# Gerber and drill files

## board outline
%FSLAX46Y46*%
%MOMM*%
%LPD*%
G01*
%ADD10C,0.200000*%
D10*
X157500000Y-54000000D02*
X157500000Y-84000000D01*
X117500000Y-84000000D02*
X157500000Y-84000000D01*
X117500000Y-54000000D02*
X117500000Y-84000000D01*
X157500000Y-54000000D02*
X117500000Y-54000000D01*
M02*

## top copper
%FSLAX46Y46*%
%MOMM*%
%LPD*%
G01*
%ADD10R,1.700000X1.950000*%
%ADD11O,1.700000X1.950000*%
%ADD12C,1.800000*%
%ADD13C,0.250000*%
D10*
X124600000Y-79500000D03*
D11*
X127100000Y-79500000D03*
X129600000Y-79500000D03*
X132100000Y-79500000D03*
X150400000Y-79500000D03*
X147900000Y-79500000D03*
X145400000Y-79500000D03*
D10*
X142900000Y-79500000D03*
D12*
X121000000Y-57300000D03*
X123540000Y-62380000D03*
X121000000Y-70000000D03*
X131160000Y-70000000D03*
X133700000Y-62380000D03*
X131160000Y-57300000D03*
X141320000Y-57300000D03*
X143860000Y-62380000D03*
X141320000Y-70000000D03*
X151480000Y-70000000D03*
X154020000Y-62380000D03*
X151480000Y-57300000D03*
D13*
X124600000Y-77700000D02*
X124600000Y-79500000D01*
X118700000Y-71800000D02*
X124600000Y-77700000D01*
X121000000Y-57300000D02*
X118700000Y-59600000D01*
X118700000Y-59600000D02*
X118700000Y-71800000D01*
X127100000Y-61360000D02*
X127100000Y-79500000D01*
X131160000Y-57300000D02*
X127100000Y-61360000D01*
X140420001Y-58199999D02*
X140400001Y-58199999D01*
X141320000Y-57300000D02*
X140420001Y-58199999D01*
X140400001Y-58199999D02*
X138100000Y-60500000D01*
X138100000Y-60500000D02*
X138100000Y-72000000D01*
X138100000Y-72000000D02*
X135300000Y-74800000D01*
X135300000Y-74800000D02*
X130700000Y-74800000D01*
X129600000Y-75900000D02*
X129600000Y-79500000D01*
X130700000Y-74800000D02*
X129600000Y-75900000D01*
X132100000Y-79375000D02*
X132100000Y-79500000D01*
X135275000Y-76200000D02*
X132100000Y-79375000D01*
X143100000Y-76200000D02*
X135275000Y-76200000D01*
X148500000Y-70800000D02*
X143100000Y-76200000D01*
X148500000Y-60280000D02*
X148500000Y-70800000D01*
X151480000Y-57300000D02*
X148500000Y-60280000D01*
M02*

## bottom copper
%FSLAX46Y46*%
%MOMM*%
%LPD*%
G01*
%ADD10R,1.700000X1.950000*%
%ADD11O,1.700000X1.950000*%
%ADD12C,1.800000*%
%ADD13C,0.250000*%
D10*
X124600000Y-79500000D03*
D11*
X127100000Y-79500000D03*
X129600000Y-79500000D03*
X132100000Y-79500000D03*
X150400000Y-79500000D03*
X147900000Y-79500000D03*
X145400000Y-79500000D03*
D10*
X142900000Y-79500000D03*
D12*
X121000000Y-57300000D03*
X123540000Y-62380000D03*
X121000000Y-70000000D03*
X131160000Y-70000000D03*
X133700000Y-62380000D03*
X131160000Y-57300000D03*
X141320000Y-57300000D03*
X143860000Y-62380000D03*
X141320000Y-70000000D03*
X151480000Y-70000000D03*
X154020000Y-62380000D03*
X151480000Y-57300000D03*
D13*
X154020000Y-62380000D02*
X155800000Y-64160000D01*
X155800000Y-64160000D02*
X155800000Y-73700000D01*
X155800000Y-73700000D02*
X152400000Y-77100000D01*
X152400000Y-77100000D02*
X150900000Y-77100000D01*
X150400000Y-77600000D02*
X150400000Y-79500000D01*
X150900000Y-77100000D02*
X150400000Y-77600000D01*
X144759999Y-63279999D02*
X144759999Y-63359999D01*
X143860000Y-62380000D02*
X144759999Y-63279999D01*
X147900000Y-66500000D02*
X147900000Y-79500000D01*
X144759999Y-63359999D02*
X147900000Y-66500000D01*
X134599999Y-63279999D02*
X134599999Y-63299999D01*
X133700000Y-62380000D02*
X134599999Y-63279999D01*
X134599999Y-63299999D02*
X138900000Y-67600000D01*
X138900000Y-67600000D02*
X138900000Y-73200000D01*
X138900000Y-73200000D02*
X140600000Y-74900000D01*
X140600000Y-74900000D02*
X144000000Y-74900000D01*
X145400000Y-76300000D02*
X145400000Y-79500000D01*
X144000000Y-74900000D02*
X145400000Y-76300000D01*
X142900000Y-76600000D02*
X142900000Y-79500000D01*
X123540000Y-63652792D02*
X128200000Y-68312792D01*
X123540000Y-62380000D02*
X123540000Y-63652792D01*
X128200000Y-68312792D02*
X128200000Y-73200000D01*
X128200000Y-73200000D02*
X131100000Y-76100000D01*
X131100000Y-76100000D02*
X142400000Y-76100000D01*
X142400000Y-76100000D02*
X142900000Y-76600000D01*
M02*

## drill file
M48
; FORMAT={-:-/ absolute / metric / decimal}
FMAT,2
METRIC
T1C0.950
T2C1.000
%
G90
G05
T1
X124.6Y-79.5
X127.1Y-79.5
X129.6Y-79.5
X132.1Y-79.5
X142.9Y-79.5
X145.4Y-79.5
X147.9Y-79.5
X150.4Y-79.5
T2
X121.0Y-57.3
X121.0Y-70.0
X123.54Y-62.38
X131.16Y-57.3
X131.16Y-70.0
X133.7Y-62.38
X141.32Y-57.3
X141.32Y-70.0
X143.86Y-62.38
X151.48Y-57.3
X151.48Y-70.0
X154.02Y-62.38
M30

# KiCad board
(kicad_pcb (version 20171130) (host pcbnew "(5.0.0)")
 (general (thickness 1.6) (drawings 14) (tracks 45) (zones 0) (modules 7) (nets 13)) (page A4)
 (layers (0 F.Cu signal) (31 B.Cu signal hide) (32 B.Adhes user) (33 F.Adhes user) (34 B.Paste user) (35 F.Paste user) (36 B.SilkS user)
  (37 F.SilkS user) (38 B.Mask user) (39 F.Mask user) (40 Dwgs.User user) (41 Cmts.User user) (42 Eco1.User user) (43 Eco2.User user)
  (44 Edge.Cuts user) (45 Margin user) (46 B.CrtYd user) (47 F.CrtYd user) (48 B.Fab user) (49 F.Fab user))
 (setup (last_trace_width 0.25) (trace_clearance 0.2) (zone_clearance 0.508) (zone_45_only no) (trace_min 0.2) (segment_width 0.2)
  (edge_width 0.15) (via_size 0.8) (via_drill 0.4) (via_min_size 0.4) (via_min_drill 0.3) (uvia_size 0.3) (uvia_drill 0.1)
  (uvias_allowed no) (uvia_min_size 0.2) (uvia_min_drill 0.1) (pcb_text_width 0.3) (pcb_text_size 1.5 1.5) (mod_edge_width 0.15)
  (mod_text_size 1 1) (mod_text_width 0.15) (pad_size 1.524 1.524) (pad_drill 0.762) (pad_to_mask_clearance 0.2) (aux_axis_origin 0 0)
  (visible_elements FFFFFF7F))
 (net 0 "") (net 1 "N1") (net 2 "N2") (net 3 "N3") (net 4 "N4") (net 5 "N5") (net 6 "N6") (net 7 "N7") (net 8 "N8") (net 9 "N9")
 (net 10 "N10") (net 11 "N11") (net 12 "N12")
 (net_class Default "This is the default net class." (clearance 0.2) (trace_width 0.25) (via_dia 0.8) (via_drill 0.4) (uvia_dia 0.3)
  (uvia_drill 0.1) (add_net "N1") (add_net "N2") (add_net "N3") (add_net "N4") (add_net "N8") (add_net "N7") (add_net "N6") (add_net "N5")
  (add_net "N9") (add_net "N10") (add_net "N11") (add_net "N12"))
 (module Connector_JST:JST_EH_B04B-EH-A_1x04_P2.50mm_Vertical (layer F.Cu) (at 124.6 79.5)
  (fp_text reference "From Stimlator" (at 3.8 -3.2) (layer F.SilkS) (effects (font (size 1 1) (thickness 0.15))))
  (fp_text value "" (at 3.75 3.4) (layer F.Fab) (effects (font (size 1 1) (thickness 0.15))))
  (pad 1 thru_hole rect (at 0 0) (size 1.7 1.95) (drill 0.95) (layers *.Cu *.Mask) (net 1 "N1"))
  (pad 2 thru_hole oval (at 2.5 0) (size 1.7 1.95) (drill 0.95) (layers *.Cu *.Mask) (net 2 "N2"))
  (pad 3 thru_hole oval (at 5 0) (size 1.7 1.95) (drill 0.95) (layers *.Cu *.Mask) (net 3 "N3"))
  (pad 4 thru_hole oval (at 7.5 0) (size 1.7 1.95) (drill 0.95) (layers *.Cu *.Mask) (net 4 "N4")))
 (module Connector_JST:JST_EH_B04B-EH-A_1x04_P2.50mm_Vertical (layer F.Cu) (at 142.9 79.5)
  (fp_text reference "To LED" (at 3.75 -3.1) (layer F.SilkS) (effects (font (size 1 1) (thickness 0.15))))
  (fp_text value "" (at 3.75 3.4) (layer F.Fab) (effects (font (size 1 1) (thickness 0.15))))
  (pad 4 thru_hole oval (at 7.5 0) (size 1.7 1.95) (drill 0.95) (layers *.Cu *.Mask) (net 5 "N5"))
  (pad 3 thru_hole oval (at 5 0) (size 1.7 1.95) (drill 0.95) (layers *.Cu *.Mask) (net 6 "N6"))
  (pad 2 thru_hole oval (at 2.5 0) (size 1.7 1.95) (drill 0.95) (layers *.Cu *.Mask) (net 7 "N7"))
  (pad 1 thru_hole rect (at 0 0) (size 1.7 1.95) (drill 0.95) (layers *.Cu *.Mask) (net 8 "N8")))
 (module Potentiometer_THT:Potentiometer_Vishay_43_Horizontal (layer F.Cu) (at 121 70 270)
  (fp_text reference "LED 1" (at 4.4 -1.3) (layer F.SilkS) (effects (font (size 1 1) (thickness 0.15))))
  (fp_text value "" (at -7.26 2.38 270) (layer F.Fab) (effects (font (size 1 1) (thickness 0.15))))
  (pad 3 thru_hole circle (at -12.7 0 270) (size 1.8 1.8) (drill 1) (layers *.Cu *.Mask) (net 1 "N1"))
  (pad 2 thru_hole circle (at -7.62 -2.54 270) (size 1.8 1.8) (drill 1) (layers *.Cu *.Mask) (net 8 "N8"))
  (pad 1 thru_hole circle (at 0 0 270) (size 1.8 1.8) (drill 1) (layers *.Cu *.Mask)))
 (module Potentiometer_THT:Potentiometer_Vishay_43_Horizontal (layer F.Cu) (at 131.16 70 270)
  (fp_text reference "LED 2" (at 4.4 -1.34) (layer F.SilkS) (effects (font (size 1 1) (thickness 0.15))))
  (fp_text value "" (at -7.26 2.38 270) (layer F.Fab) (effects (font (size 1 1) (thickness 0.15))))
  (pad 1 thru_hole circle (at 0 0 270) (size 1.8 1.8) (drill 1) (layers *.Cu *.Mask))
  (pad 2 thru_hole circle (at -7.62 -2.54 270) (size 1.8 1.8) (drill 1) (layers *.Cu *.Mask) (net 7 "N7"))
  (pad 3 thru_hole circle (at -12.7 0 270) (size 1.8 1.8) (drill 1) (layers *.Cu *.Mask) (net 2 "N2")))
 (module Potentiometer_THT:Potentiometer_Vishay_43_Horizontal (layer F.Cu) (at 141.32 70 270)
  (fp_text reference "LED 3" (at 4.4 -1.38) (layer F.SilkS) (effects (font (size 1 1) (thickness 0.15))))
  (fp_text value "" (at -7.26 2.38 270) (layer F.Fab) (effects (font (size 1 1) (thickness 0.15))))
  (pad 3 thru_hole circle (at -12.7 0 270) (size 1.8 1.8) (drill 1) (layers *.Cu *.Mask) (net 3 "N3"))
  (pad 2 thru_hole circle (at -7.62 -2.54 270) (size 1.8 1.8) (drill 1) (layers *.Cu *.Mask) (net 6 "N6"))
  (pad 1 thru_hole circle (at 0 0 270) (size 1.8 1.8) (drill 1) (layers *.Cu *.Mask)))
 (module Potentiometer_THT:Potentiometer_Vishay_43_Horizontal (layer F.Cu) (at 151.48 70 270)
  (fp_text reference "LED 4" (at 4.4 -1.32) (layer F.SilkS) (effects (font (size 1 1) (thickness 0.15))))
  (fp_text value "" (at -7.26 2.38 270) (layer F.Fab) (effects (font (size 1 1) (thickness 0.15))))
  (pad 1 thru_hole circle (at 0 0 270) (size 1.8 1.8) (drill 1) (layers *.Cu *.Mask))
  (pad 2 thru_hole circle (at -7.62 -2.54 270) (size 1.8 1.8) (drill 1) (layers *.Cu *.Mask) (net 5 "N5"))
  (pad 3 thru_hole circle (at -12.7 0 270) (size 1.8 1.8) (drill 1) (layers *.Cu *.Mask) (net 4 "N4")))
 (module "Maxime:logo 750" (layer B.Cu) (at 137.5 75.1 180)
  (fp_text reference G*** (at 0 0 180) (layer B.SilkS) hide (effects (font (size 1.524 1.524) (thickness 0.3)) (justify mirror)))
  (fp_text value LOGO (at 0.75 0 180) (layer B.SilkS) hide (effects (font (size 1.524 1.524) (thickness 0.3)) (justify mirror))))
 (gr_line (start 157.5 54) (end 157.5 84) (layer Edge.Cuts) (width 0.2))
 (gr_line (start 117.5 84) (end 157.5 84) (layer Edge.Cuts) (width 0.2))
 (gr_line (start 117.5 54) (end 117.5 84) (layer Edge.Cuts) (width 0.2))
 (gr_line (start 157.5 54) (end 117.5 54) (layer Edge.Cuts) (width 0.2))
 (segment (start 124.6 77.7) (end 124.6 79.5) (width 0.25) (layer F.Cu) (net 1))
 (segment (start 118.7 71.8) (end 124.6 77.7) (width 0.25) (layer F.Cu) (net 1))
 (segment (start 121 57.3) (end 118.7 59.6) (width 0.25) (layer F.Cu) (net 1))
 (segment (start 118.7 59.6) (end 118.7 71.8) (width 0.25) (layer F.Cu) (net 1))
 (segment (start 127.1 61.36) (end 127.1 79.5) (width 0.25) (layer F.Cu) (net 2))
 (segment (start 131.16 57.3) (end 127.1 61.36) (width 0.25) (layer F.Cu) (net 2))
 (segment (start 140.420001 58.199999) (end 140.400001 58.199999) (width 0.25) (layer F.Cu) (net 3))
 (segment (start 141.32 57.3) (end 140.420001 58.199999) (width 0.25) (layer F.Cu) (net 3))
 (segment (start 140.400001 58.199999) (end 138.1 60.5) (width 0.25) (layer F.Cu) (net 3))
 (segment (start 138.1 60.5) (end 138.1 72) (width 0.25) (layer F.Cu) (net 3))
 (segment (start 138.1 72) (end 135.3 74.8) (width 0.25) (layer F.Cu) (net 3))
 (segment (start 135.3 74.8) (end 130.7 74.8) (width 0.25) (layer F.Cu) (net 3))
 (segment (start 129.6 75.9) (end 129.6 79.5) (width 0.25) (layer F.Cu) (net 3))
 (segment (start 130.7 74.8) (end 129.6 75.9) (width 0.25) (layer F.Cu) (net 3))
 (segment (start 132.1 79.375) (end 132.1 79.5) (width 0.25) (layer F.Cu) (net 4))
 (segment (start 135.275 76.2) (end 132.1 79.375) (width 0.25) (layer F.Cu) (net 4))
 (segment (start 143.1 76.2) (end 135.275 76.2) (width 0.25) (layer F.Cu) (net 4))
 (segment (start 148.5 70.8) (end 143.1 76.2) (width 0.25) (layer F.Cu) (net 4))
 (segment (start 148.5 60.28) (end 148.5 70.8) (width 0.25) (layer F.Cu) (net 4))
 (segment (start 151.48 57.3) (end 148.5 60.28) (width 0.25) (layer F.Cu) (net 4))
 (segment (start 154.02 62.38) (end 155.8 64.16) (width 0.25) (layer B.Cu) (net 5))
 (segment (start 155.8 64.16) (end 155.8 73.7) (width 0.25) (layer B.Cu) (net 5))
 (segment (start 155.8 73.7) (end 152.4 77.1) (width 0.25) (layer B.Cu) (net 5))
 (segment (start 152.4 77.1) (end 150.9 77.1) (width 0.25) (layer B.Cu) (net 5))
 (segment (start 150.4 77.6) (end 150.4 79.5) (width 0.25) (layer B.Cu) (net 5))
 (segment (start 150.9 77.1) (end 150.4 77.6) (width 0.25) (layer B.Cu) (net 5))
 (segment (start 144.759999 63.279999) (end 144.759999 63.359999) (width 0.25) (layer B.Cu) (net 6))
 (segment (start 143.86 62.38) (end 144.759999 63.279999) (width 0.25) (layer B.Cu) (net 6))
 (segment (start 147.9 66.5) (end 147.9 79.5) (width 0.25) (layer B.Cu) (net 6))
 (segment (start 144.759999 63.359999) (end 147.9 66.5) (width 0.25) (layer B.Cu) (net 6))
 (segment (start 134.599999 63.279999) (end 134.599999 63.299999) (width 0.25) (layer B.Cu) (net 7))
 (segment (start 133.7 62.38) (end 134.599999 63.279999) (width 0.25) (layer B.Cu) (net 7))
 (segment (start 134.599999 63.299999) (end 138.9 67.6) (width 0.25) (layer B.Cu) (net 7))
 (segment (start 138.9 67.6) (end 138.9 73.2) (width 0.25) (layer B.Cu) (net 7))
 (segment (start 138.9 73.2) (end 140.6 74.9) (width 0.25) (layer B.Cu) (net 7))
 (segment (start 140.6 74.9) (end 144 74.9) (width 0.25) (layer B.Cu) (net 7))
 (segment (start 145.4 76.3) (end 145.4 79.5) (width 0.25) (layer B.Cu) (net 7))
 (segment (start 144 74.9) (end 145.4 76.3) (width 0.25) (layer B.Cu) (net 7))
 (segment (start 142.9 76.6) (end 142.9 79.5) (width 0.25) (layer B.Cu) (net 8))
 (segment (start 123.54 63.652792) (end 128.2 68.312792) (width 0.25) (layer B.Cu) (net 8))
 (segment (start 123.54 62.38) (end 123.54 63.652792) (width 0.25) (layer B.Cu) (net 8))
 (segment (start 128.2 68.312792) (end 128.2 73.2) (width 0.25) (layer B.Cu) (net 8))
 (segment (start 128.2 73.2) (end 131.1 76.1) (width 0.25) (layer B.Cu) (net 8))
 (segment (start 131.1 76.1) (end 142.4 76.1) (width 0.25) (layer B.Cu) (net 8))
 (segment (start 142.4 76.1) (end 142.9 76.6) (width 0.25) (layer B.Cu) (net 8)))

